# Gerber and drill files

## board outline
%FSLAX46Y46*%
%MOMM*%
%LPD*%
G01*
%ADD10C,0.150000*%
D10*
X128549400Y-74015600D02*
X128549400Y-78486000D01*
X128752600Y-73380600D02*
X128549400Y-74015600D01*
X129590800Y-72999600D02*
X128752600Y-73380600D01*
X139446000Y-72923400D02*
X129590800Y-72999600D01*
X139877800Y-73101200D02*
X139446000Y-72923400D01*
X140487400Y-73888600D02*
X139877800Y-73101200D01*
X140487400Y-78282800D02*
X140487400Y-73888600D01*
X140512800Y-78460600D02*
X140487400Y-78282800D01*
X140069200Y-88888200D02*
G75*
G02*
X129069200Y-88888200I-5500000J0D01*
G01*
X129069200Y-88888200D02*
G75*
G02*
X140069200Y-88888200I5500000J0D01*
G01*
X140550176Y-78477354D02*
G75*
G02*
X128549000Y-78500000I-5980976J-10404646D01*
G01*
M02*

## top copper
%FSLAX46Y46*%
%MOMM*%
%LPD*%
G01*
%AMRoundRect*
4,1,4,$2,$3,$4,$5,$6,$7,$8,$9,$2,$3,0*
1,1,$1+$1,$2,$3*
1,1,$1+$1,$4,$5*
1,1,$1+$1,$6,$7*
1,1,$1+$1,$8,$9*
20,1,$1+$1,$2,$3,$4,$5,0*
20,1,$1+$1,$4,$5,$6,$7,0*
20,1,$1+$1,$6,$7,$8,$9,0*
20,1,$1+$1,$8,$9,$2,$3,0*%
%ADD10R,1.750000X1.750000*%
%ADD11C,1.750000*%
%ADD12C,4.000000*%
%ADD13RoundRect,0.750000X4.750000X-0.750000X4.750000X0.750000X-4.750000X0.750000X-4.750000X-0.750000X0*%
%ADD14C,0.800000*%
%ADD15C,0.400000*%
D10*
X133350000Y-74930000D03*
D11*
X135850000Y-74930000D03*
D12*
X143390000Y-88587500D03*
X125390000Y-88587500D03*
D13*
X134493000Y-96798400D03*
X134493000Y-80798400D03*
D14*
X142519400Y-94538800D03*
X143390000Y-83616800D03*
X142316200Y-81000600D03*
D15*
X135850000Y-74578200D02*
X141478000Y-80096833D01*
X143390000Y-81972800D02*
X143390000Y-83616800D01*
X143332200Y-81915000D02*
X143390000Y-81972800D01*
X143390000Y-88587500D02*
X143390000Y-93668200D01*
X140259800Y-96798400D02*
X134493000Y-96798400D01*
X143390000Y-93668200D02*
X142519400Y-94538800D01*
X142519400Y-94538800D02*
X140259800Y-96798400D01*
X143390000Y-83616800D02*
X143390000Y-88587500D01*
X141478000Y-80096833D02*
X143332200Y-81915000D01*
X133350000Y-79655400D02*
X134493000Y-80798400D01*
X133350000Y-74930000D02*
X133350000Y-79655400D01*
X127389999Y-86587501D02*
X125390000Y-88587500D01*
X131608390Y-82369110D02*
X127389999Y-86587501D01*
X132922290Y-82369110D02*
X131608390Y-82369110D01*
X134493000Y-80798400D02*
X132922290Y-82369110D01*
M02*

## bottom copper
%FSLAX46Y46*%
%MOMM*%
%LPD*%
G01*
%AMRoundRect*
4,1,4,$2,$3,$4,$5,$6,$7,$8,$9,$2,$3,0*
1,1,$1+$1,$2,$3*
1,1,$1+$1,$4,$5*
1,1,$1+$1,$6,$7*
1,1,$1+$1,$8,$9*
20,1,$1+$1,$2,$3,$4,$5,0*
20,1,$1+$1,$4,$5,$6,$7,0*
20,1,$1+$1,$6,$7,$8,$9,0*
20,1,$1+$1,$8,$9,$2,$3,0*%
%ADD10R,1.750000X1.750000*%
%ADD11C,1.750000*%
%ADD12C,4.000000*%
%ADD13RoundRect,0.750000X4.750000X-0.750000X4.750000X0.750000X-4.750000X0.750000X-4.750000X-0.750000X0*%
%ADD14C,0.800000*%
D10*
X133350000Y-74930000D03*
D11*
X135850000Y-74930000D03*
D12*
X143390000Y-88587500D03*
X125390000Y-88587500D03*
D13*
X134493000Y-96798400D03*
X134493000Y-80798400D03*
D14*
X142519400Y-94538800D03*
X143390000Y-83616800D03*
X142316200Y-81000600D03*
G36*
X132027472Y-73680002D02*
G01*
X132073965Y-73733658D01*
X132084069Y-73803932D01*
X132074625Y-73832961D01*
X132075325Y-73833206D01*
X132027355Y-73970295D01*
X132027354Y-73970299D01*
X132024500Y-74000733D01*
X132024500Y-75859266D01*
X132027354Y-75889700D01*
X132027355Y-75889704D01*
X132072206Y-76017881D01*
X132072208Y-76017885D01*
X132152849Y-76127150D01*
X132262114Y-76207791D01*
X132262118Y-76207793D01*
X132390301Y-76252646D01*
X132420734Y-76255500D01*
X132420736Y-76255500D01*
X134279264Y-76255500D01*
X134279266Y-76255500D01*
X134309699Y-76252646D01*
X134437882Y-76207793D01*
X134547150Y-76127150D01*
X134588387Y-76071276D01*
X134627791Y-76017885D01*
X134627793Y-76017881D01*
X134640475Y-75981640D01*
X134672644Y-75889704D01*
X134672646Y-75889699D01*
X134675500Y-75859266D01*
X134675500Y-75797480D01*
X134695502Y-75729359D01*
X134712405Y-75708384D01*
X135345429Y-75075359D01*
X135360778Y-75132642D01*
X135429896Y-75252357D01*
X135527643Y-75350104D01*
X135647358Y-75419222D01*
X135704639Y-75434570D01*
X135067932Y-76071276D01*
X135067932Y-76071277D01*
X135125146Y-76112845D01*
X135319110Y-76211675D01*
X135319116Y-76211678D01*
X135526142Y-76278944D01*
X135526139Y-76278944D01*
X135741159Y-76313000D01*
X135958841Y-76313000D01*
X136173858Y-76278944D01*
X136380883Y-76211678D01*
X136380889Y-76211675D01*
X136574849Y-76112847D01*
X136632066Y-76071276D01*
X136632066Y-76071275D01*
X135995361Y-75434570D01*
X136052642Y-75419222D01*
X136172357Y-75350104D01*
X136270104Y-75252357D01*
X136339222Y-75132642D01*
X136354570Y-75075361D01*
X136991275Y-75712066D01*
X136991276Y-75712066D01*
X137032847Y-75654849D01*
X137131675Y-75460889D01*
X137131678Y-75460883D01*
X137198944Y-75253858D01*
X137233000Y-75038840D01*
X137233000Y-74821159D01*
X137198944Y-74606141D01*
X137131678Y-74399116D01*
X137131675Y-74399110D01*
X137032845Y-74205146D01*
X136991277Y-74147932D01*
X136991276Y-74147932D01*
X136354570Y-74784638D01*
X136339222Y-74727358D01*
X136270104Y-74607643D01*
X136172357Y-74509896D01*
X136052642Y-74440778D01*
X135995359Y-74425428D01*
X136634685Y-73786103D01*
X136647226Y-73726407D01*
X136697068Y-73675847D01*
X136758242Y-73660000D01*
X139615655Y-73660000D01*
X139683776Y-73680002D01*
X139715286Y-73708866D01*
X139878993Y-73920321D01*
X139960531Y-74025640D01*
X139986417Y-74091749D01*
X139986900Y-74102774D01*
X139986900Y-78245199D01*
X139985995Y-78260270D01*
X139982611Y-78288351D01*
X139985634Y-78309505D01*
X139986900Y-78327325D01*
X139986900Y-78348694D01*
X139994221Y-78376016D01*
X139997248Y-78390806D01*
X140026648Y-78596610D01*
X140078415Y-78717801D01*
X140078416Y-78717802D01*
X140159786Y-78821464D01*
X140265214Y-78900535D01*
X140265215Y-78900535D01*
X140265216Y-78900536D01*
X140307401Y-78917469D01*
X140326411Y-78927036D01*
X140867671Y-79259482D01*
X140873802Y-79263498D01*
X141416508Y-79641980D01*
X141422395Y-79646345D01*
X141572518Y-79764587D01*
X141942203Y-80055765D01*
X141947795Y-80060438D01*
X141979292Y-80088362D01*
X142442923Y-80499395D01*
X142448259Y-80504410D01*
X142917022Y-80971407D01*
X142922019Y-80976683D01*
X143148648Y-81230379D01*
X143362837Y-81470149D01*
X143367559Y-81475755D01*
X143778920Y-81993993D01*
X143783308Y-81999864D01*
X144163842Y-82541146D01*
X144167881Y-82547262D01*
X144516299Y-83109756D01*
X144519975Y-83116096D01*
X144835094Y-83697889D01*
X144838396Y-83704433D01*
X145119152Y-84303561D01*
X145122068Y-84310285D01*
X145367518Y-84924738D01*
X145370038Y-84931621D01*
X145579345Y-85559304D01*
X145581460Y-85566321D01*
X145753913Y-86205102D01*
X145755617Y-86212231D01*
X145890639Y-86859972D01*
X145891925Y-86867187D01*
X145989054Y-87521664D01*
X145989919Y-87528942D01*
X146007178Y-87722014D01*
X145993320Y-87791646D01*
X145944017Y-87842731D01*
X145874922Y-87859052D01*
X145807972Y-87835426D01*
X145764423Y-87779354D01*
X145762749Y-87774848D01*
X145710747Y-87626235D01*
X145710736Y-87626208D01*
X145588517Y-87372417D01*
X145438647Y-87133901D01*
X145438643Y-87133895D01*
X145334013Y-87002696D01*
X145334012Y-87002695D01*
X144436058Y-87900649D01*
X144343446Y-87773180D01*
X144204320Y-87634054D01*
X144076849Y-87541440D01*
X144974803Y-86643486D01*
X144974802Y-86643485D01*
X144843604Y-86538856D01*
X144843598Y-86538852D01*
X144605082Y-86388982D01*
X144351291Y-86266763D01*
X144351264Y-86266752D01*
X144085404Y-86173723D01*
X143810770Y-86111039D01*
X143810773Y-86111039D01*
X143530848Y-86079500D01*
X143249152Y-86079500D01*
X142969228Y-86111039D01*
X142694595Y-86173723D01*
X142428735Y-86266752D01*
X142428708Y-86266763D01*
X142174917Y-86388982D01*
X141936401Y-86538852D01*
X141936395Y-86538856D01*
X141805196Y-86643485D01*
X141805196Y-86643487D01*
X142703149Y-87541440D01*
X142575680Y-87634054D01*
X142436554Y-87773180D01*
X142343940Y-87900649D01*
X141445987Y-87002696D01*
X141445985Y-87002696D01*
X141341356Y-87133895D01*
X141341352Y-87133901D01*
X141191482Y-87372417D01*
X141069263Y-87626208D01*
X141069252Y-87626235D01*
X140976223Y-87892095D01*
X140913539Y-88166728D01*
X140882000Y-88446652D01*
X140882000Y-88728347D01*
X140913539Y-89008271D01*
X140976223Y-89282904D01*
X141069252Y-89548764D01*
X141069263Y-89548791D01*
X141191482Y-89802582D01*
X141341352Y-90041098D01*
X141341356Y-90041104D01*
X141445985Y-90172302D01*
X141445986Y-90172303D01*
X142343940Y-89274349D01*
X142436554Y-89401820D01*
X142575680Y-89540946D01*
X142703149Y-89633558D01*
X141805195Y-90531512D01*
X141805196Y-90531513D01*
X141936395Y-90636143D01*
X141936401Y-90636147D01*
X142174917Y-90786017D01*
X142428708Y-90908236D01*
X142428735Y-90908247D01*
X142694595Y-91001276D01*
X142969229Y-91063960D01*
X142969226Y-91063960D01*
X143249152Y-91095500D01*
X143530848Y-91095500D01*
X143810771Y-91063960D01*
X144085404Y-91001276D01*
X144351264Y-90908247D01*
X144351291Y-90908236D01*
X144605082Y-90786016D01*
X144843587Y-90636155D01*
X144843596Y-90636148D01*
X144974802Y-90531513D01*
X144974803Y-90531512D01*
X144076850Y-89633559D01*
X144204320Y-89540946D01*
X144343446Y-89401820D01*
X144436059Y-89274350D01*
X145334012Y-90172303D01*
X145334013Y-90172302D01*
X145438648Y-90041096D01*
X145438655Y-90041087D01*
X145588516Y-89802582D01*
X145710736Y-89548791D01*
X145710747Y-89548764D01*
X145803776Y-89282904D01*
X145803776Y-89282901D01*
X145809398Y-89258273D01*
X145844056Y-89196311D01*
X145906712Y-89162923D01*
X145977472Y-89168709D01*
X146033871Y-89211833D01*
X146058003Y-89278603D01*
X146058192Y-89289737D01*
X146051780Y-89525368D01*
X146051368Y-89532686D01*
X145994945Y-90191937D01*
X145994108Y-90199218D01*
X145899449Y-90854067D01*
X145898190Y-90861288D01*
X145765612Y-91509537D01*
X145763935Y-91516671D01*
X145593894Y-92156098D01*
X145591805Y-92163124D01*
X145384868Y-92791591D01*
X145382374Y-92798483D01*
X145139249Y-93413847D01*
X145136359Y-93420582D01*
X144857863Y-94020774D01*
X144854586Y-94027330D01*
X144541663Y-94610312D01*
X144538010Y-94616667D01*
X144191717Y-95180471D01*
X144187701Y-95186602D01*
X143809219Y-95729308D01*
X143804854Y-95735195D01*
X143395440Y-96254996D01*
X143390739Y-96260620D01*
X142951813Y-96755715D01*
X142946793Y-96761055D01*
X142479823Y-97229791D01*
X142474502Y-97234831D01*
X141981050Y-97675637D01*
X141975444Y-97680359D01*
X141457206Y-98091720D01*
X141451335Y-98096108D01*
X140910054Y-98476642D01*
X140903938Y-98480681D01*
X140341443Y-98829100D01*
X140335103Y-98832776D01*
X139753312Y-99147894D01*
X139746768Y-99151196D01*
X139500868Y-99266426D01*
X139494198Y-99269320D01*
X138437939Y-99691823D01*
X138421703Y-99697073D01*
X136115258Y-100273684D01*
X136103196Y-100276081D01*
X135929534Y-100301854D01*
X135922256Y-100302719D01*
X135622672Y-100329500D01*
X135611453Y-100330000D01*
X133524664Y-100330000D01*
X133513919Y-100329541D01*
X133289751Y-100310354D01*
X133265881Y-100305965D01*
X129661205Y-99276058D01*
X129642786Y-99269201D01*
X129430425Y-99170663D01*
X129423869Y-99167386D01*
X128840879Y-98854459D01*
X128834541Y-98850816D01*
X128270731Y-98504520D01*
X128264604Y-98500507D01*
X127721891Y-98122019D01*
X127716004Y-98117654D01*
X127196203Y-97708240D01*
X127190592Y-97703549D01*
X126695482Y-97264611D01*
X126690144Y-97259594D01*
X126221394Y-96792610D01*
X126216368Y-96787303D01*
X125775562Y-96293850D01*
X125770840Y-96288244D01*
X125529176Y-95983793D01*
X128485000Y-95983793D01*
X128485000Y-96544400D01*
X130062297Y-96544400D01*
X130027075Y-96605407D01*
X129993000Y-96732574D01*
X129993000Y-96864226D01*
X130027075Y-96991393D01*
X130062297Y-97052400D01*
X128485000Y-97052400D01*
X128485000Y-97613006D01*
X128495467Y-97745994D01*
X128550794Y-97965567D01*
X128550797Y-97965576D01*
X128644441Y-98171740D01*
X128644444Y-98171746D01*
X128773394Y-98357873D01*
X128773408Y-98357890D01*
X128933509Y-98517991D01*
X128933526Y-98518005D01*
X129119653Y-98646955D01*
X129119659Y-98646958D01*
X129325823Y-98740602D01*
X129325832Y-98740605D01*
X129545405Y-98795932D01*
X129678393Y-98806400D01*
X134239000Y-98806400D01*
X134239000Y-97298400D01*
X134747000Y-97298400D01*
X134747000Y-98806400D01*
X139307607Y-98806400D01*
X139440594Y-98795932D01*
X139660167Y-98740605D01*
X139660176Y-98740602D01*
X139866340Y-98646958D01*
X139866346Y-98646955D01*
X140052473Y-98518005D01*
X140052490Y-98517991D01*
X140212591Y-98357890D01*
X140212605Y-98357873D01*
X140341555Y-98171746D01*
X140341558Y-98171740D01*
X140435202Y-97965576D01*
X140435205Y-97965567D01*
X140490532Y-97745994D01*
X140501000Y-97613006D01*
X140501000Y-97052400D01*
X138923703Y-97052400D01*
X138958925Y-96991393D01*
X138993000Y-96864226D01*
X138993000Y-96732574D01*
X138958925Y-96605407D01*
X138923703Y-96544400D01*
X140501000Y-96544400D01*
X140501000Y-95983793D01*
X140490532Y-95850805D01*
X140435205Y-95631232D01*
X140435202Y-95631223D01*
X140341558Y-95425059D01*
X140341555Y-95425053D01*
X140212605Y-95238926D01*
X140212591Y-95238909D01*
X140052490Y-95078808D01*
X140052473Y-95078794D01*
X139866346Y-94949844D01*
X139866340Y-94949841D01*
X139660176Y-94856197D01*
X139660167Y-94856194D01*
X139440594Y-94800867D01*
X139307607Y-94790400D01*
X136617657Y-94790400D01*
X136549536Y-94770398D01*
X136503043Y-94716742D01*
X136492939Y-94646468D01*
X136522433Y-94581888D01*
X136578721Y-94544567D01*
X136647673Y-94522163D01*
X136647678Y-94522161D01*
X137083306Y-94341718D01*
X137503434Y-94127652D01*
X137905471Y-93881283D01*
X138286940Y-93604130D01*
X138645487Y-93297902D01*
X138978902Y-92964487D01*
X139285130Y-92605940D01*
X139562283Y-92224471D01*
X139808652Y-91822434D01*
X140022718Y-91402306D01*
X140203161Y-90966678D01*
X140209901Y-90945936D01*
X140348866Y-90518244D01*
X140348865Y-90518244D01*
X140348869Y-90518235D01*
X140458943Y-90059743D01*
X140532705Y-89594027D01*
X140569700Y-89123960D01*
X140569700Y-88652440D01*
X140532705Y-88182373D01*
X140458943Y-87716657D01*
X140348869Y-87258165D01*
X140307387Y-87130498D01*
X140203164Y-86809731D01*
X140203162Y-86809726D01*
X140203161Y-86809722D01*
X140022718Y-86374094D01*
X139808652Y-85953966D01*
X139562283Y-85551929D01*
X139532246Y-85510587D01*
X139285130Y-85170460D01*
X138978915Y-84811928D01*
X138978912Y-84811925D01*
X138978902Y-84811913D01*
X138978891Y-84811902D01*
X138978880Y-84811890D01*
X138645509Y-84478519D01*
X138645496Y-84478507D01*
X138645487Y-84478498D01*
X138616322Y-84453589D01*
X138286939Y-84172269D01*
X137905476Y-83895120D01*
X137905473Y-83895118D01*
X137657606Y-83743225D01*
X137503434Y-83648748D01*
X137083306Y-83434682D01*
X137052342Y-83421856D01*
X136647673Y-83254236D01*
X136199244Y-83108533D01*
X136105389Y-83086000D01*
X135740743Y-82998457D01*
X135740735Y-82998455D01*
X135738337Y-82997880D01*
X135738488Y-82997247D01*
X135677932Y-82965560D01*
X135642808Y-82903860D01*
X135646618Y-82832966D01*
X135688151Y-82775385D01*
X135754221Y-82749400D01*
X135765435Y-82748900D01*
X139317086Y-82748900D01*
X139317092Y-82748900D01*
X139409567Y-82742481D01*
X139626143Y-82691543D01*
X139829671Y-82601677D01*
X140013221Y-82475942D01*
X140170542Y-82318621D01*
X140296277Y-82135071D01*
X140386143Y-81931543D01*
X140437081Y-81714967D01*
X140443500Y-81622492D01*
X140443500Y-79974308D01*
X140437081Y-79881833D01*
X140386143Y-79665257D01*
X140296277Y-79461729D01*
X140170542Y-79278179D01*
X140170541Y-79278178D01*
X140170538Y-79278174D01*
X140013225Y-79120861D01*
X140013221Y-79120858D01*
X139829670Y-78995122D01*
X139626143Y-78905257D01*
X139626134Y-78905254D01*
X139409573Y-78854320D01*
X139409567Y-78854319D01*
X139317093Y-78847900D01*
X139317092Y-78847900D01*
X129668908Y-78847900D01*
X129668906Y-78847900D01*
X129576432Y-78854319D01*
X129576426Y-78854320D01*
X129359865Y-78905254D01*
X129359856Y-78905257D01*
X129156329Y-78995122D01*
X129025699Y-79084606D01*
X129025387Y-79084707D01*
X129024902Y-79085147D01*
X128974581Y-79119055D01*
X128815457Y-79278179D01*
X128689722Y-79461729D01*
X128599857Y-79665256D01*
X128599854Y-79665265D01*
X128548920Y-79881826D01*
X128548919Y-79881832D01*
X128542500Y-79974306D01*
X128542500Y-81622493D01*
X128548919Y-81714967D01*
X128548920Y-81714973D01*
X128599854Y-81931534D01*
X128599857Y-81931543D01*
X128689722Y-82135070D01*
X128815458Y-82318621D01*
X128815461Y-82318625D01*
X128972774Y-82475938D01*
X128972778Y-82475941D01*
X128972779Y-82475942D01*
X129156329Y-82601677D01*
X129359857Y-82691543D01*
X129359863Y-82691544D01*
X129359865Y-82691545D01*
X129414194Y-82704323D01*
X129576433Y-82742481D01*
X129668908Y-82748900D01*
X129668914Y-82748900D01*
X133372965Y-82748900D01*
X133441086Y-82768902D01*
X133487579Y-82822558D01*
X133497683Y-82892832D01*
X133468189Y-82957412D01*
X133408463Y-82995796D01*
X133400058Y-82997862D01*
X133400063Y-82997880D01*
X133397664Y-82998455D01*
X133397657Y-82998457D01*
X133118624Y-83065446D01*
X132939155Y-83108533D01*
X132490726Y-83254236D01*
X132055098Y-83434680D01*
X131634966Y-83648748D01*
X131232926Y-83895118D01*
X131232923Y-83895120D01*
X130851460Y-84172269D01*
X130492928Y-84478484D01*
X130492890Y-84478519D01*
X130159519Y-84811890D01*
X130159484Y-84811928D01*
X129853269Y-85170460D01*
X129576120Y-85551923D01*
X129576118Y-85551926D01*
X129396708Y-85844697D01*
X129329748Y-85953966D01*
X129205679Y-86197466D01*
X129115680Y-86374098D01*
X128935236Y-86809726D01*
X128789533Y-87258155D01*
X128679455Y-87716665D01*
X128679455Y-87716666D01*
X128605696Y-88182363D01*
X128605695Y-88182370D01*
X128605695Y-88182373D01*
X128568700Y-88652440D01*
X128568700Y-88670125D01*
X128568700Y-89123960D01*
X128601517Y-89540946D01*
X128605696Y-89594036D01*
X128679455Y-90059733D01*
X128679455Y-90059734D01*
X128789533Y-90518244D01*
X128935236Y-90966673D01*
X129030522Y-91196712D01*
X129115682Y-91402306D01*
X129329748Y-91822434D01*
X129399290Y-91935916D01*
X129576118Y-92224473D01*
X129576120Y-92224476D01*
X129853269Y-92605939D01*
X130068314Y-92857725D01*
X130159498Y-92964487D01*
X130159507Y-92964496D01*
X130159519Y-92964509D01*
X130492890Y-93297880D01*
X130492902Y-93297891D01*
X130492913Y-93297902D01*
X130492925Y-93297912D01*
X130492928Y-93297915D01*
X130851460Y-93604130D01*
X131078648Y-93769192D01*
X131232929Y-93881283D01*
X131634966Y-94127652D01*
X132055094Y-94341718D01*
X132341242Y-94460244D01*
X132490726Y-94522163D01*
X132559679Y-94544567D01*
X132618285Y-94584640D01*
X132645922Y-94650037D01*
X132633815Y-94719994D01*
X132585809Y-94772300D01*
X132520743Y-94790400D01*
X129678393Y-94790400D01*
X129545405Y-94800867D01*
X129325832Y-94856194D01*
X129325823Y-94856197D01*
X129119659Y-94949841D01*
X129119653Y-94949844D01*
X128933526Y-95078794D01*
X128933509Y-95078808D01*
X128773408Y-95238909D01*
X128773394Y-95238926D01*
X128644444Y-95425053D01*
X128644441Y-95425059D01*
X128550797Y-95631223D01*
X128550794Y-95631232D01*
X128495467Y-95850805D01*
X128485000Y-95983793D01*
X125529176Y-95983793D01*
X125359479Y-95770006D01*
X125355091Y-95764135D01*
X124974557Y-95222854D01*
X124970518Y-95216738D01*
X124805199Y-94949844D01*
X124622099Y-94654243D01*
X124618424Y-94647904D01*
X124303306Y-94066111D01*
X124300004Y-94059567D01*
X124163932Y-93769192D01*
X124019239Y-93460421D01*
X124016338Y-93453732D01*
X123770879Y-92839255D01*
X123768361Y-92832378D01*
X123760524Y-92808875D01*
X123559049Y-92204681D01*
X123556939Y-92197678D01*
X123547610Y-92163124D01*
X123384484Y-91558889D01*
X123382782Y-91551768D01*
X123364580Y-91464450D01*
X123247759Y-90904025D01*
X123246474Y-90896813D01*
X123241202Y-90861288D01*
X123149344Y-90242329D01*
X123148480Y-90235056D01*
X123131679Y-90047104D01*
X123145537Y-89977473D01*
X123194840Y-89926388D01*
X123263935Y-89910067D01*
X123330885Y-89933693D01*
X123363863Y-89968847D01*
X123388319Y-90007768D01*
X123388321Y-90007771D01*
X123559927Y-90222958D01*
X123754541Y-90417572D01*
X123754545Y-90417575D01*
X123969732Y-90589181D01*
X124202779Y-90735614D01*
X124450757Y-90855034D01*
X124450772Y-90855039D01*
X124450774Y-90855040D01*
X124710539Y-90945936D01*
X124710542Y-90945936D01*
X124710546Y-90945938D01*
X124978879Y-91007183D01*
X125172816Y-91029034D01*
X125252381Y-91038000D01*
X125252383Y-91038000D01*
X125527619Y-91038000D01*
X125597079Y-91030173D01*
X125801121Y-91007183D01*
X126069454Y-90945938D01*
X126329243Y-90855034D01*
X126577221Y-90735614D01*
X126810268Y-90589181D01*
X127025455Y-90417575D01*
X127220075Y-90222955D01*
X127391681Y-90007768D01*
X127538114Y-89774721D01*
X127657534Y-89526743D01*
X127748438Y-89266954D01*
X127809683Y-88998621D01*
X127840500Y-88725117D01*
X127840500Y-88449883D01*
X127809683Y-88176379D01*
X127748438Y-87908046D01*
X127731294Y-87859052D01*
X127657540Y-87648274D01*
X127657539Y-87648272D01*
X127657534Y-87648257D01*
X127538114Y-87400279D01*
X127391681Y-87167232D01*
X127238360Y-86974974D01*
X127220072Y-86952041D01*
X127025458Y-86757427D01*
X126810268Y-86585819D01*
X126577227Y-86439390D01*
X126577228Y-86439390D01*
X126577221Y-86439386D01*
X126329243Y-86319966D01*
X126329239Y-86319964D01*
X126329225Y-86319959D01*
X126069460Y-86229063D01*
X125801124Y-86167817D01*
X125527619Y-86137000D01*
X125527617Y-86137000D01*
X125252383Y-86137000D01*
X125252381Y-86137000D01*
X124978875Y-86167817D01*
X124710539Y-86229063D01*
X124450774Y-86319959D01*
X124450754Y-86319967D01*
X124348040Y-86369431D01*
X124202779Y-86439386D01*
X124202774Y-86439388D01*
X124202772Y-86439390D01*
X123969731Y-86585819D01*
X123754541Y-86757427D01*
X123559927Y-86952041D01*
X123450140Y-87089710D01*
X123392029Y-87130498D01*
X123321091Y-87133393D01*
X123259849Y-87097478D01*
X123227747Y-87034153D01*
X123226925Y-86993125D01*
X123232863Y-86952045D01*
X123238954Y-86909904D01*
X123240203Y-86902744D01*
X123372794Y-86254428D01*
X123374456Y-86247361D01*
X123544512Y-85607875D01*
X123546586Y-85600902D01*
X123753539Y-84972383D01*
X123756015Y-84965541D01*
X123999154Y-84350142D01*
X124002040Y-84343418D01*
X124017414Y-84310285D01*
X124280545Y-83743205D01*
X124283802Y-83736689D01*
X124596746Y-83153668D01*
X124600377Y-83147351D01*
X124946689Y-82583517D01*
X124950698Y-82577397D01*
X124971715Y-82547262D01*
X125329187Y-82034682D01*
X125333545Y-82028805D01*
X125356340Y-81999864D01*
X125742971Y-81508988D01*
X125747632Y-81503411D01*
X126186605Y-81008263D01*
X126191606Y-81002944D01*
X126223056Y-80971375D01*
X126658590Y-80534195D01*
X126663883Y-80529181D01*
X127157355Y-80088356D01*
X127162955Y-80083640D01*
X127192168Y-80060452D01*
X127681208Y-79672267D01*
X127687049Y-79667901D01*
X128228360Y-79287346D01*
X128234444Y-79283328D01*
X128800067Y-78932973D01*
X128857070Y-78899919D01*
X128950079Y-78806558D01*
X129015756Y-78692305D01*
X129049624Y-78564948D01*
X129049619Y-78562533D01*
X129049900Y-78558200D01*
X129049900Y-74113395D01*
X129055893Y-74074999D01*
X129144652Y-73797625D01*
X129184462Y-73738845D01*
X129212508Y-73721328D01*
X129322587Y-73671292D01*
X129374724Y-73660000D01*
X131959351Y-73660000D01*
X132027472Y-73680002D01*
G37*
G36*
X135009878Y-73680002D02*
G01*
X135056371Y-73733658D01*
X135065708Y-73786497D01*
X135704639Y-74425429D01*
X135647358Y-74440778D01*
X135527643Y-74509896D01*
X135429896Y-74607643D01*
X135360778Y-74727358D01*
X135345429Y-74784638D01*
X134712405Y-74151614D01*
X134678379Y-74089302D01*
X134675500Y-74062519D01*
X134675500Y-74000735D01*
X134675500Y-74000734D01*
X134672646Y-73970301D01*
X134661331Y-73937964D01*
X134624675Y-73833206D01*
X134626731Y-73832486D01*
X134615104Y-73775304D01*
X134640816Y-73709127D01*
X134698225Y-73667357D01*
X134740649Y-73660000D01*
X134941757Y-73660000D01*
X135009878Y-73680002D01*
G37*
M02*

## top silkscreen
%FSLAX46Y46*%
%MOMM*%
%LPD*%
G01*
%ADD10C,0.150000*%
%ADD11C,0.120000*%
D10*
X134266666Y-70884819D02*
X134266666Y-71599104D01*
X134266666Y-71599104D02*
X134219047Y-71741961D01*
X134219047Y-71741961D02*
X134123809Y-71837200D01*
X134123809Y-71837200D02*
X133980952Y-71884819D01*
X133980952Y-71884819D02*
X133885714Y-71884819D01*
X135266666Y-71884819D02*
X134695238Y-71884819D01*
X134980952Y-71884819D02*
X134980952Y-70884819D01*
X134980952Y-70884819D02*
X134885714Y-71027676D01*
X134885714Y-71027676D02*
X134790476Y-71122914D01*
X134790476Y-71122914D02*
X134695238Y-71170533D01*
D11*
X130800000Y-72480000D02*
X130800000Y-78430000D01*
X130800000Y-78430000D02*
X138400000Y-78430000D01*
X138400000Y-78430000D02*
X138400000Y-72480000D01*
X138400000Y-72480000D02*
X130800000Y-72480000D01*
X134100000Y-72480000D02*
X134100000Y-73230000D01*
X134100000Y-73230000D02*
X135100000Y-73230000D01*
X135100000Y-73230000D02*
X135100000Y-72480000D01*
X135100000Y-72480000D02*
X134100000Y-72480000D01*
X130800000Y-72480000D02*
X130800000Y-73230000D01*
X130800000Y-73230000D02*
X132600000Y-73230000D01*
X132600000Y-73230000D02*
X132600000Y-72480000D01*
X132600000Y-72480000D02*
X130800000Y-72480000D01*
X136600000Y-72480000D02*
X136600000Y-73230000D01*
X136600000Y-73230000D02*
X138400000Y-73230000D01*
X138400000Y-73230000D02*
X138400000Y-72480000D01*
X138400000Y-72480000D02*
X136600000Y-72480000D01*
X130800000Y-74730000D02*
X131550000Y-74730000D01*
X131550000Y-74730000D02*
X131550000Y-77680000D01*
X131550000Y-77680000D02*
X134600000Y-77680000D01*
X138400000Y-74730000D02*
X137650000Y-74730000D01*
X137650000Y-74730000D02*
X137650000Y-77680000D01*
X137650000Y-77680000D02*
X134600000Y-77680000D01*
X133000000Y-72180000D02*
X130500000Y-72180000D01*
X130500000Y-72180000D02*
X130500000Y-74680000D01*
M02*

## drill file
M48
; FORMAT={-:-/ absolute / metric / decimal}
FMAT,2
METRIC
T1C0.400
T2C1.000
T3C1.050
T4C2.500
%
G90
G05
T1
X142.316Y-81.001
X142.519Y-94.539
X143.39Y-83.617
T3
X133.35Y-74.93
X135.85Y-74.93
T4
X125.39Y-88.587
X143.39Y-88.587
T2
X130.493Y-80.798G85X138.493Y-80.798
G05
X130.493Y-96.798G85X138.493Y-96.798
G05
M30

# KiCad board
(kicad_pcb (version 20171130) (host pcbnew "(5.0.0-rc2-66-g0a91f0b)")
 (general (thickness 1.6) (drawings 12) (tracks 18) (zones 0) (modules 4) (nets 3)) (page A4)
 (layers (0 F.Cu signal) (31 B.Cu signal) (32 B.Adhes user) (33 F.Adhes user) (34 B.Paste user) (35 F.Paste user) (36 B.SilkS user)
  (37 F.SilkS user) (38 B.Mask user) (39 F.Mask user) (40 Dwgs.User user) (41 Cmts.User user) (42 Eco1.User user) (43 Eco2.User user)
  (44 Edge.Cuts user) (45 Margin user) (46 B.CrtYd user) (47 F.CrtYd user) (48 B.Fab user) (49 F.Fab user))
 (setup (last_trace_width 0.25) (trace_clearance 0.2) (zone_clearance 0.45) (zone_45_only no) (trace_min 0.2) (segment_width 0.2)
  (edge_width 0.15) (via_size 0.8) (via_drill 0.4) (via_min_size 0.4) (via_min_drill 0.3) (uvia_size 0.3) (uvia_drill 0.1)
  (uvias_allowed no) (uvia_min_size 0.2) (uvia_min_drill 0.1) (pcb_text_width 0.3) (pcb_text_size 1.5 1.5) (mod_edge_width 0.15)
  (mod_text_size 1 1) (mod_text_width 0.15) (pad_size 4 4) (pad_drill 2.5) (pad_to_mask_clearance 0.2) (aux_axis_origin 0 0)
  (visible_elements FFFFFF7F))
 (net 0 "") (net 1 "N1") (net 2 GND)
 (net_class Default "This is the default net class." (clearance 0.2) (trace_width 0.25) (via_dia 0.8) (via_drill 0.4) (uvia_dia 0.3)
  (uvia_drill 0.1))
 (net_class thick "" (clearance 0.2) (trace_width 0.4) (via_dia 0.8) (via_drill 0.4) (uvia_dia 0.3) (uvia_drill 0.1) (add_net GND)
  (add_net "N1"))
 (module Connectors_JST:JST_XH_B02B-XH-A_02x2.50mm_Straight (layer F.Cu) (at 133.35 74.93)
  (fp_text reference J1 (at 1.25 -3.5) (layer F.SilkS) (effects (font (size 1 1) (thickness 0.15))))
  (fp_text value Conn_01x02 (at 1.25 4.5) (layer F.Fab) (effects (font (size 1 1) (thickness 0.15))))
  (fp_line (start -2.55 -2.45) (end -2.55 3.5) (layer F.SilkS) (width 0.12))
  (fp_line (start -2.55 3.5) (end 5.05 3.5) (layer F.SilkS) (width 0.12))
  (fp_line (start 5.05 3.5) (end 5.05 -2.45) (layer F.SilkS) (width 0.12))
  (fp_line (start 5.05 -2.45) (end -2.55 -2.45) (layer F.SilkS) (width 0.12))
  (fp_line (start 0.75 -2.45) (end 0.75 -1.7) (layer F.SilkS) (width 0.12))
  (fp_line (start 0.75 -1.7) (end 1.75 -1.7) (layer F.SilkS) (width 0.12))
  (fp_line (start 1.75 -1.7) (end 1.75 -2.45) (layer F.SilkS) (width 0.12))
  (fp_line (start 1.75 -2.45) (end 0.75 -2.45) (layer F.SilkS) (width 0.12))
  (fp_line (start -2.55 -2.45) (end -2.55 -1.7) (layer F.SilkS) (width 0.12))
  (fp_line (start -2.55 -1.7) (end -0.75 -1.7) (layer F.SilkS) (width 0.12))
  (fp_line (start -0.75 -1.7) (end -0.75 -2.45) (layer F.SilkS) (width 0.12))
  (fp_line (start -0.75 -2.45) (end -2.55 -2.45) (layer F.SilkS) (width 0.12))
  (fp_line (start 3.25 -2.45) (end 3.25 -1.7) (layer F.SilkS) (width 0.12))
  (fp_line (start 3.25 -1.7) (end 5.05 -1.7) (layer F.SilkS) (width 0.12))
  (fp_line (start 5.05 -1.7) (end 5.05 -2.45) (layer F.SilkS) (width 0.12))
  (fp_line (start 5.05 -2.45) (end 3.25 -2.45) (layer F.SilkS) (width 0.12))
  (fp_line (start -2.55 -0.2) (end -1.8 -0.2) (layer F.SilkS) (width 0.12))
  (fp_line (start -1.8 -0.2) (end -1.8 2.75) (layer F.SilkS) (width 0.12))
  (fp_line (start -1.8 2.75) (end 1.25 2.75) (layer F.SilkS) (width 0.12))
  (fp_line (start 5.05 -0.2) (end 4.3 -0.2) (layer F.SilkS) (width 0.12))
  (fp_line (start 4.3 -0.2) (end 4.3 2.75) (layer F.SilkS) (width 0.12))
  (fp_line (start 4.3 2.75) (end 1.25 2.75) (layer F.SilkS) (width 0.12))
  (fp_line (start -0.35 -2.75) (end -2.85 -2.75) (layer F.SilkS) (width 0.12))
  (fp_line (start -2.85 -2.75) (end -2.85 -0.25) (layer F.SilkS) (width 0.12))
  (pad 1 thru_hole rect (at 0 0) (size 1.75 1.75) (drill 1.05) (layers *.Cu *.Mask) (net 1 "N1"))
  (pad 2 thru_hole circle (at 2.5 0) (size 1.75 1.75) (drill 1.05) (layers *.Cu *.Mask) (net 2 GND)))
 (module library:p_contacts (layer F.Cu) (at 134.39 88.5875)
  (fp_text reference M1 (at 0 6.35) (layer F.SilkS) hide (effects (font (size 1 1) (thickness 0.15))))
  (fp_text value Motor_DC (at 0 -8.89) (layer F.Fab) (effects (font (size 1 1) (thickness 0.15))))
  (pad 2 thru_hole circle (at 9 0) (size 4 4) (drill 2.5) (layers *.Mask F.Cu) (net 2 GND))
  (pad 1 thru_hole circle (at -9 0) (size 4 4) (drill 2.5) (layers *.Mask F.Cu) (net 1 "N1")))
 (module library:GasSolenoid (layer F.Cu) (at 134.493 88.7984 90)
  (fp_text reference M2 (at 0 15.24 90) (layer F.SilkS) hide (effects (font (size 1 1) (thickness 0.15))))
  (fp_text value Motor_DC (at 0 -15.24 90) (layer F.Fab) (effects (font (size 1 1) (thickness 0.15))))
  (pad 2 thru_hole roundrect (at -8 0 90) (size 3 11) (drill oval 1 9) (layers *.Mask F.Cu) (roundrect_rratio 0.25) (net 2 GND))
  (pad 1 thru_hole roundrect (at 8 0 90) (size 3 11) (drill oval 1 9) (layers *.Mask F.Cu) (roundrect_rratio 0.25) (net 1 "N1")))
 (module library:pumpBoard (layer F.Cu) (at 134.62 88.9)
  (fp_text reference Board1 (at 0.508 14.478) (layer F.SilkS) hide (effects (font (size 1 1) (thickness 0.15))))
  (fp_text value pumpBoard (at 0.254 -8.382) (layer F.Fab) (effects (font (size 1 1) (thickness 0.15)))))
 (gr_line (start 128.5494 74.0156) (end 128.5494 78.486) (layer Edge.Cuts) (width 0.15))
 (gr_line (start 128.7526 73.3806) (end 128.5494 74.0156) (layer Edge.Cuts) (width 0.15))
 (gr_line (start 129.5908 72.9996) (end 128.7526 73.3806) (layer Edge.Cuts) (width 0.15))
 (gr_line (start 139.446 72.9234) (end 129.5908 72.9996) (layer Edge.Cuts) (width 0.15))
 (gr_line (start 139.8778 73.1012) (end 139.446 72.9234) (layer Edge.Cuts) (width 0.15))
 (gr_line (start 140.4874 73.8886) (end 139.8778 73.1012) (layer Edge.Cuts) (width 0.15))
 (gr_line (start 140.4874 78.2828) (end 140.4874 73.8886) (layer Edge.Cuts) (width 0.15))
 (gr_line (start 140.5128 78.4606) (end 140.4874 78.2828) (layer Edge.Cuts) (width 0.15))
 (gr_circle (center 134.5692 88.8882) (end 140.0692 88.8882) (layer Edge.Cuts) (width 0.15))
 (gr_arc (start 134.5692 88.882) (end 128.549 78.5) (angle -300) (layer Edge.Cuts) (width 0.15))
 (segment (start 135.85 74.5782) (end 141.478 80.096833) (width 0.4) (layer F.Cu) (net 2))
 (segment (start 143.39 81.9728) (end 143.39 83.6168) (width 0.4) (layer F.Cu) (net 2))
 (segment (start 143.3322 81.915) (end 143.39 81.9728) (width 0.4) (layer F.Cu) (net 2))
 (segment (start 143.39 88.5875) (end 143.39 93.6682) (width 0.4) (layer F.Cu) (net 2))
 (segment (start 140.2598 96.7984) (end 134.493 96.7984) (width 0.4) (layer F.Cu) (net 2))
 (segment (start 143.39 93.6682) (end 142.5194 94.5388) (width 0.4) (layer F.Cu) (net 2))
 (segment (start 142.5194 94.5388) (end 140.2598 96.7984) (width 0.4) (layer F.Cu) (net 2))
 (via (at 142.5194 94.5388) (size 0.8) (drill 0.4) (layers F.Cu B.Cu) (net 2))
 (segment (start 143.39 83.6168) (end 143.39 88.5875) (width 0.4) (layer F.Cu) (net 2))
 (via (at 143.39 83.6168) (size 0.8) (drill 0.4) (layers F.Cu B.Cu) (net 2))
 (segment (start 141.478 80.096833) (end 143.3322 81.915) (width 0.4) (layer F.Cu) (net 2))
 (via (at 142.3162 81.0006) (size 0.8) (drill 0.4) (layers F.Cu B.Cu) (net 2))
 (segment (start 133.35 79.6554) (end 134.493 80.7984) (width 0.4) (layer F.Cu) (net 1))
 (segment (start 133.35 74.93) (end 133.35 79.6554) (width 0.4) (layer F.Cu) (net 1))
 (segment (start 127.389999 86.587501) (end 125.39 88.5875) (width 0.4) (layer F.Cu) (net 1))
 (segment (start 131.60839 82.36911) (end 127.389999 86.587501) (width 0.4) (layer F.Cu) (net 1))
 (segment (start 132.92229 82.36911) (end 131.60839 82.36911) (width 0.4) (layer F.Cu) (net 1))
 (segment (start 134.493 80.7984) (end 132.92229 82.36911) (width 0.4) (layer F.Cu) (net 1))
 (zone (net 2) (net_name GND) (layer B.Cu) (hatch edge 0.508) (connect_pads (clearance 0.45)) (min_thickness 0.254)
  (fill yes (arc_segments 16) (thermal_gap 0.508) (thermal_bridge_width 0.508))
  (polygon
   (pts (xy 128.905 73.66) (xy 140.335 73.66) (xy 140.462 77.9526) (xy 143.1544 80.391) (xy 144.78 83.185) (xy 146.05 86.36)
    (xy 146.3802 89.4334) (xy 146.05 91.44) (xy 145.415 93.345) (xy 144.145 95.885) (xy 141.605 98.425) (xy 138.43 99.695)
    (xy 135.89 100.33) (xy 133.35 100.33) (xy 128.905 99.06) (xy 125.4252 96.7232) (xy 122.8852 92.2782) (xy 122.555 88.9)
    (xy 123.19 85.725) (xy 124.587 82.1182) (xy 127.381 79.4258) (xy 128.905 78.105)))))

